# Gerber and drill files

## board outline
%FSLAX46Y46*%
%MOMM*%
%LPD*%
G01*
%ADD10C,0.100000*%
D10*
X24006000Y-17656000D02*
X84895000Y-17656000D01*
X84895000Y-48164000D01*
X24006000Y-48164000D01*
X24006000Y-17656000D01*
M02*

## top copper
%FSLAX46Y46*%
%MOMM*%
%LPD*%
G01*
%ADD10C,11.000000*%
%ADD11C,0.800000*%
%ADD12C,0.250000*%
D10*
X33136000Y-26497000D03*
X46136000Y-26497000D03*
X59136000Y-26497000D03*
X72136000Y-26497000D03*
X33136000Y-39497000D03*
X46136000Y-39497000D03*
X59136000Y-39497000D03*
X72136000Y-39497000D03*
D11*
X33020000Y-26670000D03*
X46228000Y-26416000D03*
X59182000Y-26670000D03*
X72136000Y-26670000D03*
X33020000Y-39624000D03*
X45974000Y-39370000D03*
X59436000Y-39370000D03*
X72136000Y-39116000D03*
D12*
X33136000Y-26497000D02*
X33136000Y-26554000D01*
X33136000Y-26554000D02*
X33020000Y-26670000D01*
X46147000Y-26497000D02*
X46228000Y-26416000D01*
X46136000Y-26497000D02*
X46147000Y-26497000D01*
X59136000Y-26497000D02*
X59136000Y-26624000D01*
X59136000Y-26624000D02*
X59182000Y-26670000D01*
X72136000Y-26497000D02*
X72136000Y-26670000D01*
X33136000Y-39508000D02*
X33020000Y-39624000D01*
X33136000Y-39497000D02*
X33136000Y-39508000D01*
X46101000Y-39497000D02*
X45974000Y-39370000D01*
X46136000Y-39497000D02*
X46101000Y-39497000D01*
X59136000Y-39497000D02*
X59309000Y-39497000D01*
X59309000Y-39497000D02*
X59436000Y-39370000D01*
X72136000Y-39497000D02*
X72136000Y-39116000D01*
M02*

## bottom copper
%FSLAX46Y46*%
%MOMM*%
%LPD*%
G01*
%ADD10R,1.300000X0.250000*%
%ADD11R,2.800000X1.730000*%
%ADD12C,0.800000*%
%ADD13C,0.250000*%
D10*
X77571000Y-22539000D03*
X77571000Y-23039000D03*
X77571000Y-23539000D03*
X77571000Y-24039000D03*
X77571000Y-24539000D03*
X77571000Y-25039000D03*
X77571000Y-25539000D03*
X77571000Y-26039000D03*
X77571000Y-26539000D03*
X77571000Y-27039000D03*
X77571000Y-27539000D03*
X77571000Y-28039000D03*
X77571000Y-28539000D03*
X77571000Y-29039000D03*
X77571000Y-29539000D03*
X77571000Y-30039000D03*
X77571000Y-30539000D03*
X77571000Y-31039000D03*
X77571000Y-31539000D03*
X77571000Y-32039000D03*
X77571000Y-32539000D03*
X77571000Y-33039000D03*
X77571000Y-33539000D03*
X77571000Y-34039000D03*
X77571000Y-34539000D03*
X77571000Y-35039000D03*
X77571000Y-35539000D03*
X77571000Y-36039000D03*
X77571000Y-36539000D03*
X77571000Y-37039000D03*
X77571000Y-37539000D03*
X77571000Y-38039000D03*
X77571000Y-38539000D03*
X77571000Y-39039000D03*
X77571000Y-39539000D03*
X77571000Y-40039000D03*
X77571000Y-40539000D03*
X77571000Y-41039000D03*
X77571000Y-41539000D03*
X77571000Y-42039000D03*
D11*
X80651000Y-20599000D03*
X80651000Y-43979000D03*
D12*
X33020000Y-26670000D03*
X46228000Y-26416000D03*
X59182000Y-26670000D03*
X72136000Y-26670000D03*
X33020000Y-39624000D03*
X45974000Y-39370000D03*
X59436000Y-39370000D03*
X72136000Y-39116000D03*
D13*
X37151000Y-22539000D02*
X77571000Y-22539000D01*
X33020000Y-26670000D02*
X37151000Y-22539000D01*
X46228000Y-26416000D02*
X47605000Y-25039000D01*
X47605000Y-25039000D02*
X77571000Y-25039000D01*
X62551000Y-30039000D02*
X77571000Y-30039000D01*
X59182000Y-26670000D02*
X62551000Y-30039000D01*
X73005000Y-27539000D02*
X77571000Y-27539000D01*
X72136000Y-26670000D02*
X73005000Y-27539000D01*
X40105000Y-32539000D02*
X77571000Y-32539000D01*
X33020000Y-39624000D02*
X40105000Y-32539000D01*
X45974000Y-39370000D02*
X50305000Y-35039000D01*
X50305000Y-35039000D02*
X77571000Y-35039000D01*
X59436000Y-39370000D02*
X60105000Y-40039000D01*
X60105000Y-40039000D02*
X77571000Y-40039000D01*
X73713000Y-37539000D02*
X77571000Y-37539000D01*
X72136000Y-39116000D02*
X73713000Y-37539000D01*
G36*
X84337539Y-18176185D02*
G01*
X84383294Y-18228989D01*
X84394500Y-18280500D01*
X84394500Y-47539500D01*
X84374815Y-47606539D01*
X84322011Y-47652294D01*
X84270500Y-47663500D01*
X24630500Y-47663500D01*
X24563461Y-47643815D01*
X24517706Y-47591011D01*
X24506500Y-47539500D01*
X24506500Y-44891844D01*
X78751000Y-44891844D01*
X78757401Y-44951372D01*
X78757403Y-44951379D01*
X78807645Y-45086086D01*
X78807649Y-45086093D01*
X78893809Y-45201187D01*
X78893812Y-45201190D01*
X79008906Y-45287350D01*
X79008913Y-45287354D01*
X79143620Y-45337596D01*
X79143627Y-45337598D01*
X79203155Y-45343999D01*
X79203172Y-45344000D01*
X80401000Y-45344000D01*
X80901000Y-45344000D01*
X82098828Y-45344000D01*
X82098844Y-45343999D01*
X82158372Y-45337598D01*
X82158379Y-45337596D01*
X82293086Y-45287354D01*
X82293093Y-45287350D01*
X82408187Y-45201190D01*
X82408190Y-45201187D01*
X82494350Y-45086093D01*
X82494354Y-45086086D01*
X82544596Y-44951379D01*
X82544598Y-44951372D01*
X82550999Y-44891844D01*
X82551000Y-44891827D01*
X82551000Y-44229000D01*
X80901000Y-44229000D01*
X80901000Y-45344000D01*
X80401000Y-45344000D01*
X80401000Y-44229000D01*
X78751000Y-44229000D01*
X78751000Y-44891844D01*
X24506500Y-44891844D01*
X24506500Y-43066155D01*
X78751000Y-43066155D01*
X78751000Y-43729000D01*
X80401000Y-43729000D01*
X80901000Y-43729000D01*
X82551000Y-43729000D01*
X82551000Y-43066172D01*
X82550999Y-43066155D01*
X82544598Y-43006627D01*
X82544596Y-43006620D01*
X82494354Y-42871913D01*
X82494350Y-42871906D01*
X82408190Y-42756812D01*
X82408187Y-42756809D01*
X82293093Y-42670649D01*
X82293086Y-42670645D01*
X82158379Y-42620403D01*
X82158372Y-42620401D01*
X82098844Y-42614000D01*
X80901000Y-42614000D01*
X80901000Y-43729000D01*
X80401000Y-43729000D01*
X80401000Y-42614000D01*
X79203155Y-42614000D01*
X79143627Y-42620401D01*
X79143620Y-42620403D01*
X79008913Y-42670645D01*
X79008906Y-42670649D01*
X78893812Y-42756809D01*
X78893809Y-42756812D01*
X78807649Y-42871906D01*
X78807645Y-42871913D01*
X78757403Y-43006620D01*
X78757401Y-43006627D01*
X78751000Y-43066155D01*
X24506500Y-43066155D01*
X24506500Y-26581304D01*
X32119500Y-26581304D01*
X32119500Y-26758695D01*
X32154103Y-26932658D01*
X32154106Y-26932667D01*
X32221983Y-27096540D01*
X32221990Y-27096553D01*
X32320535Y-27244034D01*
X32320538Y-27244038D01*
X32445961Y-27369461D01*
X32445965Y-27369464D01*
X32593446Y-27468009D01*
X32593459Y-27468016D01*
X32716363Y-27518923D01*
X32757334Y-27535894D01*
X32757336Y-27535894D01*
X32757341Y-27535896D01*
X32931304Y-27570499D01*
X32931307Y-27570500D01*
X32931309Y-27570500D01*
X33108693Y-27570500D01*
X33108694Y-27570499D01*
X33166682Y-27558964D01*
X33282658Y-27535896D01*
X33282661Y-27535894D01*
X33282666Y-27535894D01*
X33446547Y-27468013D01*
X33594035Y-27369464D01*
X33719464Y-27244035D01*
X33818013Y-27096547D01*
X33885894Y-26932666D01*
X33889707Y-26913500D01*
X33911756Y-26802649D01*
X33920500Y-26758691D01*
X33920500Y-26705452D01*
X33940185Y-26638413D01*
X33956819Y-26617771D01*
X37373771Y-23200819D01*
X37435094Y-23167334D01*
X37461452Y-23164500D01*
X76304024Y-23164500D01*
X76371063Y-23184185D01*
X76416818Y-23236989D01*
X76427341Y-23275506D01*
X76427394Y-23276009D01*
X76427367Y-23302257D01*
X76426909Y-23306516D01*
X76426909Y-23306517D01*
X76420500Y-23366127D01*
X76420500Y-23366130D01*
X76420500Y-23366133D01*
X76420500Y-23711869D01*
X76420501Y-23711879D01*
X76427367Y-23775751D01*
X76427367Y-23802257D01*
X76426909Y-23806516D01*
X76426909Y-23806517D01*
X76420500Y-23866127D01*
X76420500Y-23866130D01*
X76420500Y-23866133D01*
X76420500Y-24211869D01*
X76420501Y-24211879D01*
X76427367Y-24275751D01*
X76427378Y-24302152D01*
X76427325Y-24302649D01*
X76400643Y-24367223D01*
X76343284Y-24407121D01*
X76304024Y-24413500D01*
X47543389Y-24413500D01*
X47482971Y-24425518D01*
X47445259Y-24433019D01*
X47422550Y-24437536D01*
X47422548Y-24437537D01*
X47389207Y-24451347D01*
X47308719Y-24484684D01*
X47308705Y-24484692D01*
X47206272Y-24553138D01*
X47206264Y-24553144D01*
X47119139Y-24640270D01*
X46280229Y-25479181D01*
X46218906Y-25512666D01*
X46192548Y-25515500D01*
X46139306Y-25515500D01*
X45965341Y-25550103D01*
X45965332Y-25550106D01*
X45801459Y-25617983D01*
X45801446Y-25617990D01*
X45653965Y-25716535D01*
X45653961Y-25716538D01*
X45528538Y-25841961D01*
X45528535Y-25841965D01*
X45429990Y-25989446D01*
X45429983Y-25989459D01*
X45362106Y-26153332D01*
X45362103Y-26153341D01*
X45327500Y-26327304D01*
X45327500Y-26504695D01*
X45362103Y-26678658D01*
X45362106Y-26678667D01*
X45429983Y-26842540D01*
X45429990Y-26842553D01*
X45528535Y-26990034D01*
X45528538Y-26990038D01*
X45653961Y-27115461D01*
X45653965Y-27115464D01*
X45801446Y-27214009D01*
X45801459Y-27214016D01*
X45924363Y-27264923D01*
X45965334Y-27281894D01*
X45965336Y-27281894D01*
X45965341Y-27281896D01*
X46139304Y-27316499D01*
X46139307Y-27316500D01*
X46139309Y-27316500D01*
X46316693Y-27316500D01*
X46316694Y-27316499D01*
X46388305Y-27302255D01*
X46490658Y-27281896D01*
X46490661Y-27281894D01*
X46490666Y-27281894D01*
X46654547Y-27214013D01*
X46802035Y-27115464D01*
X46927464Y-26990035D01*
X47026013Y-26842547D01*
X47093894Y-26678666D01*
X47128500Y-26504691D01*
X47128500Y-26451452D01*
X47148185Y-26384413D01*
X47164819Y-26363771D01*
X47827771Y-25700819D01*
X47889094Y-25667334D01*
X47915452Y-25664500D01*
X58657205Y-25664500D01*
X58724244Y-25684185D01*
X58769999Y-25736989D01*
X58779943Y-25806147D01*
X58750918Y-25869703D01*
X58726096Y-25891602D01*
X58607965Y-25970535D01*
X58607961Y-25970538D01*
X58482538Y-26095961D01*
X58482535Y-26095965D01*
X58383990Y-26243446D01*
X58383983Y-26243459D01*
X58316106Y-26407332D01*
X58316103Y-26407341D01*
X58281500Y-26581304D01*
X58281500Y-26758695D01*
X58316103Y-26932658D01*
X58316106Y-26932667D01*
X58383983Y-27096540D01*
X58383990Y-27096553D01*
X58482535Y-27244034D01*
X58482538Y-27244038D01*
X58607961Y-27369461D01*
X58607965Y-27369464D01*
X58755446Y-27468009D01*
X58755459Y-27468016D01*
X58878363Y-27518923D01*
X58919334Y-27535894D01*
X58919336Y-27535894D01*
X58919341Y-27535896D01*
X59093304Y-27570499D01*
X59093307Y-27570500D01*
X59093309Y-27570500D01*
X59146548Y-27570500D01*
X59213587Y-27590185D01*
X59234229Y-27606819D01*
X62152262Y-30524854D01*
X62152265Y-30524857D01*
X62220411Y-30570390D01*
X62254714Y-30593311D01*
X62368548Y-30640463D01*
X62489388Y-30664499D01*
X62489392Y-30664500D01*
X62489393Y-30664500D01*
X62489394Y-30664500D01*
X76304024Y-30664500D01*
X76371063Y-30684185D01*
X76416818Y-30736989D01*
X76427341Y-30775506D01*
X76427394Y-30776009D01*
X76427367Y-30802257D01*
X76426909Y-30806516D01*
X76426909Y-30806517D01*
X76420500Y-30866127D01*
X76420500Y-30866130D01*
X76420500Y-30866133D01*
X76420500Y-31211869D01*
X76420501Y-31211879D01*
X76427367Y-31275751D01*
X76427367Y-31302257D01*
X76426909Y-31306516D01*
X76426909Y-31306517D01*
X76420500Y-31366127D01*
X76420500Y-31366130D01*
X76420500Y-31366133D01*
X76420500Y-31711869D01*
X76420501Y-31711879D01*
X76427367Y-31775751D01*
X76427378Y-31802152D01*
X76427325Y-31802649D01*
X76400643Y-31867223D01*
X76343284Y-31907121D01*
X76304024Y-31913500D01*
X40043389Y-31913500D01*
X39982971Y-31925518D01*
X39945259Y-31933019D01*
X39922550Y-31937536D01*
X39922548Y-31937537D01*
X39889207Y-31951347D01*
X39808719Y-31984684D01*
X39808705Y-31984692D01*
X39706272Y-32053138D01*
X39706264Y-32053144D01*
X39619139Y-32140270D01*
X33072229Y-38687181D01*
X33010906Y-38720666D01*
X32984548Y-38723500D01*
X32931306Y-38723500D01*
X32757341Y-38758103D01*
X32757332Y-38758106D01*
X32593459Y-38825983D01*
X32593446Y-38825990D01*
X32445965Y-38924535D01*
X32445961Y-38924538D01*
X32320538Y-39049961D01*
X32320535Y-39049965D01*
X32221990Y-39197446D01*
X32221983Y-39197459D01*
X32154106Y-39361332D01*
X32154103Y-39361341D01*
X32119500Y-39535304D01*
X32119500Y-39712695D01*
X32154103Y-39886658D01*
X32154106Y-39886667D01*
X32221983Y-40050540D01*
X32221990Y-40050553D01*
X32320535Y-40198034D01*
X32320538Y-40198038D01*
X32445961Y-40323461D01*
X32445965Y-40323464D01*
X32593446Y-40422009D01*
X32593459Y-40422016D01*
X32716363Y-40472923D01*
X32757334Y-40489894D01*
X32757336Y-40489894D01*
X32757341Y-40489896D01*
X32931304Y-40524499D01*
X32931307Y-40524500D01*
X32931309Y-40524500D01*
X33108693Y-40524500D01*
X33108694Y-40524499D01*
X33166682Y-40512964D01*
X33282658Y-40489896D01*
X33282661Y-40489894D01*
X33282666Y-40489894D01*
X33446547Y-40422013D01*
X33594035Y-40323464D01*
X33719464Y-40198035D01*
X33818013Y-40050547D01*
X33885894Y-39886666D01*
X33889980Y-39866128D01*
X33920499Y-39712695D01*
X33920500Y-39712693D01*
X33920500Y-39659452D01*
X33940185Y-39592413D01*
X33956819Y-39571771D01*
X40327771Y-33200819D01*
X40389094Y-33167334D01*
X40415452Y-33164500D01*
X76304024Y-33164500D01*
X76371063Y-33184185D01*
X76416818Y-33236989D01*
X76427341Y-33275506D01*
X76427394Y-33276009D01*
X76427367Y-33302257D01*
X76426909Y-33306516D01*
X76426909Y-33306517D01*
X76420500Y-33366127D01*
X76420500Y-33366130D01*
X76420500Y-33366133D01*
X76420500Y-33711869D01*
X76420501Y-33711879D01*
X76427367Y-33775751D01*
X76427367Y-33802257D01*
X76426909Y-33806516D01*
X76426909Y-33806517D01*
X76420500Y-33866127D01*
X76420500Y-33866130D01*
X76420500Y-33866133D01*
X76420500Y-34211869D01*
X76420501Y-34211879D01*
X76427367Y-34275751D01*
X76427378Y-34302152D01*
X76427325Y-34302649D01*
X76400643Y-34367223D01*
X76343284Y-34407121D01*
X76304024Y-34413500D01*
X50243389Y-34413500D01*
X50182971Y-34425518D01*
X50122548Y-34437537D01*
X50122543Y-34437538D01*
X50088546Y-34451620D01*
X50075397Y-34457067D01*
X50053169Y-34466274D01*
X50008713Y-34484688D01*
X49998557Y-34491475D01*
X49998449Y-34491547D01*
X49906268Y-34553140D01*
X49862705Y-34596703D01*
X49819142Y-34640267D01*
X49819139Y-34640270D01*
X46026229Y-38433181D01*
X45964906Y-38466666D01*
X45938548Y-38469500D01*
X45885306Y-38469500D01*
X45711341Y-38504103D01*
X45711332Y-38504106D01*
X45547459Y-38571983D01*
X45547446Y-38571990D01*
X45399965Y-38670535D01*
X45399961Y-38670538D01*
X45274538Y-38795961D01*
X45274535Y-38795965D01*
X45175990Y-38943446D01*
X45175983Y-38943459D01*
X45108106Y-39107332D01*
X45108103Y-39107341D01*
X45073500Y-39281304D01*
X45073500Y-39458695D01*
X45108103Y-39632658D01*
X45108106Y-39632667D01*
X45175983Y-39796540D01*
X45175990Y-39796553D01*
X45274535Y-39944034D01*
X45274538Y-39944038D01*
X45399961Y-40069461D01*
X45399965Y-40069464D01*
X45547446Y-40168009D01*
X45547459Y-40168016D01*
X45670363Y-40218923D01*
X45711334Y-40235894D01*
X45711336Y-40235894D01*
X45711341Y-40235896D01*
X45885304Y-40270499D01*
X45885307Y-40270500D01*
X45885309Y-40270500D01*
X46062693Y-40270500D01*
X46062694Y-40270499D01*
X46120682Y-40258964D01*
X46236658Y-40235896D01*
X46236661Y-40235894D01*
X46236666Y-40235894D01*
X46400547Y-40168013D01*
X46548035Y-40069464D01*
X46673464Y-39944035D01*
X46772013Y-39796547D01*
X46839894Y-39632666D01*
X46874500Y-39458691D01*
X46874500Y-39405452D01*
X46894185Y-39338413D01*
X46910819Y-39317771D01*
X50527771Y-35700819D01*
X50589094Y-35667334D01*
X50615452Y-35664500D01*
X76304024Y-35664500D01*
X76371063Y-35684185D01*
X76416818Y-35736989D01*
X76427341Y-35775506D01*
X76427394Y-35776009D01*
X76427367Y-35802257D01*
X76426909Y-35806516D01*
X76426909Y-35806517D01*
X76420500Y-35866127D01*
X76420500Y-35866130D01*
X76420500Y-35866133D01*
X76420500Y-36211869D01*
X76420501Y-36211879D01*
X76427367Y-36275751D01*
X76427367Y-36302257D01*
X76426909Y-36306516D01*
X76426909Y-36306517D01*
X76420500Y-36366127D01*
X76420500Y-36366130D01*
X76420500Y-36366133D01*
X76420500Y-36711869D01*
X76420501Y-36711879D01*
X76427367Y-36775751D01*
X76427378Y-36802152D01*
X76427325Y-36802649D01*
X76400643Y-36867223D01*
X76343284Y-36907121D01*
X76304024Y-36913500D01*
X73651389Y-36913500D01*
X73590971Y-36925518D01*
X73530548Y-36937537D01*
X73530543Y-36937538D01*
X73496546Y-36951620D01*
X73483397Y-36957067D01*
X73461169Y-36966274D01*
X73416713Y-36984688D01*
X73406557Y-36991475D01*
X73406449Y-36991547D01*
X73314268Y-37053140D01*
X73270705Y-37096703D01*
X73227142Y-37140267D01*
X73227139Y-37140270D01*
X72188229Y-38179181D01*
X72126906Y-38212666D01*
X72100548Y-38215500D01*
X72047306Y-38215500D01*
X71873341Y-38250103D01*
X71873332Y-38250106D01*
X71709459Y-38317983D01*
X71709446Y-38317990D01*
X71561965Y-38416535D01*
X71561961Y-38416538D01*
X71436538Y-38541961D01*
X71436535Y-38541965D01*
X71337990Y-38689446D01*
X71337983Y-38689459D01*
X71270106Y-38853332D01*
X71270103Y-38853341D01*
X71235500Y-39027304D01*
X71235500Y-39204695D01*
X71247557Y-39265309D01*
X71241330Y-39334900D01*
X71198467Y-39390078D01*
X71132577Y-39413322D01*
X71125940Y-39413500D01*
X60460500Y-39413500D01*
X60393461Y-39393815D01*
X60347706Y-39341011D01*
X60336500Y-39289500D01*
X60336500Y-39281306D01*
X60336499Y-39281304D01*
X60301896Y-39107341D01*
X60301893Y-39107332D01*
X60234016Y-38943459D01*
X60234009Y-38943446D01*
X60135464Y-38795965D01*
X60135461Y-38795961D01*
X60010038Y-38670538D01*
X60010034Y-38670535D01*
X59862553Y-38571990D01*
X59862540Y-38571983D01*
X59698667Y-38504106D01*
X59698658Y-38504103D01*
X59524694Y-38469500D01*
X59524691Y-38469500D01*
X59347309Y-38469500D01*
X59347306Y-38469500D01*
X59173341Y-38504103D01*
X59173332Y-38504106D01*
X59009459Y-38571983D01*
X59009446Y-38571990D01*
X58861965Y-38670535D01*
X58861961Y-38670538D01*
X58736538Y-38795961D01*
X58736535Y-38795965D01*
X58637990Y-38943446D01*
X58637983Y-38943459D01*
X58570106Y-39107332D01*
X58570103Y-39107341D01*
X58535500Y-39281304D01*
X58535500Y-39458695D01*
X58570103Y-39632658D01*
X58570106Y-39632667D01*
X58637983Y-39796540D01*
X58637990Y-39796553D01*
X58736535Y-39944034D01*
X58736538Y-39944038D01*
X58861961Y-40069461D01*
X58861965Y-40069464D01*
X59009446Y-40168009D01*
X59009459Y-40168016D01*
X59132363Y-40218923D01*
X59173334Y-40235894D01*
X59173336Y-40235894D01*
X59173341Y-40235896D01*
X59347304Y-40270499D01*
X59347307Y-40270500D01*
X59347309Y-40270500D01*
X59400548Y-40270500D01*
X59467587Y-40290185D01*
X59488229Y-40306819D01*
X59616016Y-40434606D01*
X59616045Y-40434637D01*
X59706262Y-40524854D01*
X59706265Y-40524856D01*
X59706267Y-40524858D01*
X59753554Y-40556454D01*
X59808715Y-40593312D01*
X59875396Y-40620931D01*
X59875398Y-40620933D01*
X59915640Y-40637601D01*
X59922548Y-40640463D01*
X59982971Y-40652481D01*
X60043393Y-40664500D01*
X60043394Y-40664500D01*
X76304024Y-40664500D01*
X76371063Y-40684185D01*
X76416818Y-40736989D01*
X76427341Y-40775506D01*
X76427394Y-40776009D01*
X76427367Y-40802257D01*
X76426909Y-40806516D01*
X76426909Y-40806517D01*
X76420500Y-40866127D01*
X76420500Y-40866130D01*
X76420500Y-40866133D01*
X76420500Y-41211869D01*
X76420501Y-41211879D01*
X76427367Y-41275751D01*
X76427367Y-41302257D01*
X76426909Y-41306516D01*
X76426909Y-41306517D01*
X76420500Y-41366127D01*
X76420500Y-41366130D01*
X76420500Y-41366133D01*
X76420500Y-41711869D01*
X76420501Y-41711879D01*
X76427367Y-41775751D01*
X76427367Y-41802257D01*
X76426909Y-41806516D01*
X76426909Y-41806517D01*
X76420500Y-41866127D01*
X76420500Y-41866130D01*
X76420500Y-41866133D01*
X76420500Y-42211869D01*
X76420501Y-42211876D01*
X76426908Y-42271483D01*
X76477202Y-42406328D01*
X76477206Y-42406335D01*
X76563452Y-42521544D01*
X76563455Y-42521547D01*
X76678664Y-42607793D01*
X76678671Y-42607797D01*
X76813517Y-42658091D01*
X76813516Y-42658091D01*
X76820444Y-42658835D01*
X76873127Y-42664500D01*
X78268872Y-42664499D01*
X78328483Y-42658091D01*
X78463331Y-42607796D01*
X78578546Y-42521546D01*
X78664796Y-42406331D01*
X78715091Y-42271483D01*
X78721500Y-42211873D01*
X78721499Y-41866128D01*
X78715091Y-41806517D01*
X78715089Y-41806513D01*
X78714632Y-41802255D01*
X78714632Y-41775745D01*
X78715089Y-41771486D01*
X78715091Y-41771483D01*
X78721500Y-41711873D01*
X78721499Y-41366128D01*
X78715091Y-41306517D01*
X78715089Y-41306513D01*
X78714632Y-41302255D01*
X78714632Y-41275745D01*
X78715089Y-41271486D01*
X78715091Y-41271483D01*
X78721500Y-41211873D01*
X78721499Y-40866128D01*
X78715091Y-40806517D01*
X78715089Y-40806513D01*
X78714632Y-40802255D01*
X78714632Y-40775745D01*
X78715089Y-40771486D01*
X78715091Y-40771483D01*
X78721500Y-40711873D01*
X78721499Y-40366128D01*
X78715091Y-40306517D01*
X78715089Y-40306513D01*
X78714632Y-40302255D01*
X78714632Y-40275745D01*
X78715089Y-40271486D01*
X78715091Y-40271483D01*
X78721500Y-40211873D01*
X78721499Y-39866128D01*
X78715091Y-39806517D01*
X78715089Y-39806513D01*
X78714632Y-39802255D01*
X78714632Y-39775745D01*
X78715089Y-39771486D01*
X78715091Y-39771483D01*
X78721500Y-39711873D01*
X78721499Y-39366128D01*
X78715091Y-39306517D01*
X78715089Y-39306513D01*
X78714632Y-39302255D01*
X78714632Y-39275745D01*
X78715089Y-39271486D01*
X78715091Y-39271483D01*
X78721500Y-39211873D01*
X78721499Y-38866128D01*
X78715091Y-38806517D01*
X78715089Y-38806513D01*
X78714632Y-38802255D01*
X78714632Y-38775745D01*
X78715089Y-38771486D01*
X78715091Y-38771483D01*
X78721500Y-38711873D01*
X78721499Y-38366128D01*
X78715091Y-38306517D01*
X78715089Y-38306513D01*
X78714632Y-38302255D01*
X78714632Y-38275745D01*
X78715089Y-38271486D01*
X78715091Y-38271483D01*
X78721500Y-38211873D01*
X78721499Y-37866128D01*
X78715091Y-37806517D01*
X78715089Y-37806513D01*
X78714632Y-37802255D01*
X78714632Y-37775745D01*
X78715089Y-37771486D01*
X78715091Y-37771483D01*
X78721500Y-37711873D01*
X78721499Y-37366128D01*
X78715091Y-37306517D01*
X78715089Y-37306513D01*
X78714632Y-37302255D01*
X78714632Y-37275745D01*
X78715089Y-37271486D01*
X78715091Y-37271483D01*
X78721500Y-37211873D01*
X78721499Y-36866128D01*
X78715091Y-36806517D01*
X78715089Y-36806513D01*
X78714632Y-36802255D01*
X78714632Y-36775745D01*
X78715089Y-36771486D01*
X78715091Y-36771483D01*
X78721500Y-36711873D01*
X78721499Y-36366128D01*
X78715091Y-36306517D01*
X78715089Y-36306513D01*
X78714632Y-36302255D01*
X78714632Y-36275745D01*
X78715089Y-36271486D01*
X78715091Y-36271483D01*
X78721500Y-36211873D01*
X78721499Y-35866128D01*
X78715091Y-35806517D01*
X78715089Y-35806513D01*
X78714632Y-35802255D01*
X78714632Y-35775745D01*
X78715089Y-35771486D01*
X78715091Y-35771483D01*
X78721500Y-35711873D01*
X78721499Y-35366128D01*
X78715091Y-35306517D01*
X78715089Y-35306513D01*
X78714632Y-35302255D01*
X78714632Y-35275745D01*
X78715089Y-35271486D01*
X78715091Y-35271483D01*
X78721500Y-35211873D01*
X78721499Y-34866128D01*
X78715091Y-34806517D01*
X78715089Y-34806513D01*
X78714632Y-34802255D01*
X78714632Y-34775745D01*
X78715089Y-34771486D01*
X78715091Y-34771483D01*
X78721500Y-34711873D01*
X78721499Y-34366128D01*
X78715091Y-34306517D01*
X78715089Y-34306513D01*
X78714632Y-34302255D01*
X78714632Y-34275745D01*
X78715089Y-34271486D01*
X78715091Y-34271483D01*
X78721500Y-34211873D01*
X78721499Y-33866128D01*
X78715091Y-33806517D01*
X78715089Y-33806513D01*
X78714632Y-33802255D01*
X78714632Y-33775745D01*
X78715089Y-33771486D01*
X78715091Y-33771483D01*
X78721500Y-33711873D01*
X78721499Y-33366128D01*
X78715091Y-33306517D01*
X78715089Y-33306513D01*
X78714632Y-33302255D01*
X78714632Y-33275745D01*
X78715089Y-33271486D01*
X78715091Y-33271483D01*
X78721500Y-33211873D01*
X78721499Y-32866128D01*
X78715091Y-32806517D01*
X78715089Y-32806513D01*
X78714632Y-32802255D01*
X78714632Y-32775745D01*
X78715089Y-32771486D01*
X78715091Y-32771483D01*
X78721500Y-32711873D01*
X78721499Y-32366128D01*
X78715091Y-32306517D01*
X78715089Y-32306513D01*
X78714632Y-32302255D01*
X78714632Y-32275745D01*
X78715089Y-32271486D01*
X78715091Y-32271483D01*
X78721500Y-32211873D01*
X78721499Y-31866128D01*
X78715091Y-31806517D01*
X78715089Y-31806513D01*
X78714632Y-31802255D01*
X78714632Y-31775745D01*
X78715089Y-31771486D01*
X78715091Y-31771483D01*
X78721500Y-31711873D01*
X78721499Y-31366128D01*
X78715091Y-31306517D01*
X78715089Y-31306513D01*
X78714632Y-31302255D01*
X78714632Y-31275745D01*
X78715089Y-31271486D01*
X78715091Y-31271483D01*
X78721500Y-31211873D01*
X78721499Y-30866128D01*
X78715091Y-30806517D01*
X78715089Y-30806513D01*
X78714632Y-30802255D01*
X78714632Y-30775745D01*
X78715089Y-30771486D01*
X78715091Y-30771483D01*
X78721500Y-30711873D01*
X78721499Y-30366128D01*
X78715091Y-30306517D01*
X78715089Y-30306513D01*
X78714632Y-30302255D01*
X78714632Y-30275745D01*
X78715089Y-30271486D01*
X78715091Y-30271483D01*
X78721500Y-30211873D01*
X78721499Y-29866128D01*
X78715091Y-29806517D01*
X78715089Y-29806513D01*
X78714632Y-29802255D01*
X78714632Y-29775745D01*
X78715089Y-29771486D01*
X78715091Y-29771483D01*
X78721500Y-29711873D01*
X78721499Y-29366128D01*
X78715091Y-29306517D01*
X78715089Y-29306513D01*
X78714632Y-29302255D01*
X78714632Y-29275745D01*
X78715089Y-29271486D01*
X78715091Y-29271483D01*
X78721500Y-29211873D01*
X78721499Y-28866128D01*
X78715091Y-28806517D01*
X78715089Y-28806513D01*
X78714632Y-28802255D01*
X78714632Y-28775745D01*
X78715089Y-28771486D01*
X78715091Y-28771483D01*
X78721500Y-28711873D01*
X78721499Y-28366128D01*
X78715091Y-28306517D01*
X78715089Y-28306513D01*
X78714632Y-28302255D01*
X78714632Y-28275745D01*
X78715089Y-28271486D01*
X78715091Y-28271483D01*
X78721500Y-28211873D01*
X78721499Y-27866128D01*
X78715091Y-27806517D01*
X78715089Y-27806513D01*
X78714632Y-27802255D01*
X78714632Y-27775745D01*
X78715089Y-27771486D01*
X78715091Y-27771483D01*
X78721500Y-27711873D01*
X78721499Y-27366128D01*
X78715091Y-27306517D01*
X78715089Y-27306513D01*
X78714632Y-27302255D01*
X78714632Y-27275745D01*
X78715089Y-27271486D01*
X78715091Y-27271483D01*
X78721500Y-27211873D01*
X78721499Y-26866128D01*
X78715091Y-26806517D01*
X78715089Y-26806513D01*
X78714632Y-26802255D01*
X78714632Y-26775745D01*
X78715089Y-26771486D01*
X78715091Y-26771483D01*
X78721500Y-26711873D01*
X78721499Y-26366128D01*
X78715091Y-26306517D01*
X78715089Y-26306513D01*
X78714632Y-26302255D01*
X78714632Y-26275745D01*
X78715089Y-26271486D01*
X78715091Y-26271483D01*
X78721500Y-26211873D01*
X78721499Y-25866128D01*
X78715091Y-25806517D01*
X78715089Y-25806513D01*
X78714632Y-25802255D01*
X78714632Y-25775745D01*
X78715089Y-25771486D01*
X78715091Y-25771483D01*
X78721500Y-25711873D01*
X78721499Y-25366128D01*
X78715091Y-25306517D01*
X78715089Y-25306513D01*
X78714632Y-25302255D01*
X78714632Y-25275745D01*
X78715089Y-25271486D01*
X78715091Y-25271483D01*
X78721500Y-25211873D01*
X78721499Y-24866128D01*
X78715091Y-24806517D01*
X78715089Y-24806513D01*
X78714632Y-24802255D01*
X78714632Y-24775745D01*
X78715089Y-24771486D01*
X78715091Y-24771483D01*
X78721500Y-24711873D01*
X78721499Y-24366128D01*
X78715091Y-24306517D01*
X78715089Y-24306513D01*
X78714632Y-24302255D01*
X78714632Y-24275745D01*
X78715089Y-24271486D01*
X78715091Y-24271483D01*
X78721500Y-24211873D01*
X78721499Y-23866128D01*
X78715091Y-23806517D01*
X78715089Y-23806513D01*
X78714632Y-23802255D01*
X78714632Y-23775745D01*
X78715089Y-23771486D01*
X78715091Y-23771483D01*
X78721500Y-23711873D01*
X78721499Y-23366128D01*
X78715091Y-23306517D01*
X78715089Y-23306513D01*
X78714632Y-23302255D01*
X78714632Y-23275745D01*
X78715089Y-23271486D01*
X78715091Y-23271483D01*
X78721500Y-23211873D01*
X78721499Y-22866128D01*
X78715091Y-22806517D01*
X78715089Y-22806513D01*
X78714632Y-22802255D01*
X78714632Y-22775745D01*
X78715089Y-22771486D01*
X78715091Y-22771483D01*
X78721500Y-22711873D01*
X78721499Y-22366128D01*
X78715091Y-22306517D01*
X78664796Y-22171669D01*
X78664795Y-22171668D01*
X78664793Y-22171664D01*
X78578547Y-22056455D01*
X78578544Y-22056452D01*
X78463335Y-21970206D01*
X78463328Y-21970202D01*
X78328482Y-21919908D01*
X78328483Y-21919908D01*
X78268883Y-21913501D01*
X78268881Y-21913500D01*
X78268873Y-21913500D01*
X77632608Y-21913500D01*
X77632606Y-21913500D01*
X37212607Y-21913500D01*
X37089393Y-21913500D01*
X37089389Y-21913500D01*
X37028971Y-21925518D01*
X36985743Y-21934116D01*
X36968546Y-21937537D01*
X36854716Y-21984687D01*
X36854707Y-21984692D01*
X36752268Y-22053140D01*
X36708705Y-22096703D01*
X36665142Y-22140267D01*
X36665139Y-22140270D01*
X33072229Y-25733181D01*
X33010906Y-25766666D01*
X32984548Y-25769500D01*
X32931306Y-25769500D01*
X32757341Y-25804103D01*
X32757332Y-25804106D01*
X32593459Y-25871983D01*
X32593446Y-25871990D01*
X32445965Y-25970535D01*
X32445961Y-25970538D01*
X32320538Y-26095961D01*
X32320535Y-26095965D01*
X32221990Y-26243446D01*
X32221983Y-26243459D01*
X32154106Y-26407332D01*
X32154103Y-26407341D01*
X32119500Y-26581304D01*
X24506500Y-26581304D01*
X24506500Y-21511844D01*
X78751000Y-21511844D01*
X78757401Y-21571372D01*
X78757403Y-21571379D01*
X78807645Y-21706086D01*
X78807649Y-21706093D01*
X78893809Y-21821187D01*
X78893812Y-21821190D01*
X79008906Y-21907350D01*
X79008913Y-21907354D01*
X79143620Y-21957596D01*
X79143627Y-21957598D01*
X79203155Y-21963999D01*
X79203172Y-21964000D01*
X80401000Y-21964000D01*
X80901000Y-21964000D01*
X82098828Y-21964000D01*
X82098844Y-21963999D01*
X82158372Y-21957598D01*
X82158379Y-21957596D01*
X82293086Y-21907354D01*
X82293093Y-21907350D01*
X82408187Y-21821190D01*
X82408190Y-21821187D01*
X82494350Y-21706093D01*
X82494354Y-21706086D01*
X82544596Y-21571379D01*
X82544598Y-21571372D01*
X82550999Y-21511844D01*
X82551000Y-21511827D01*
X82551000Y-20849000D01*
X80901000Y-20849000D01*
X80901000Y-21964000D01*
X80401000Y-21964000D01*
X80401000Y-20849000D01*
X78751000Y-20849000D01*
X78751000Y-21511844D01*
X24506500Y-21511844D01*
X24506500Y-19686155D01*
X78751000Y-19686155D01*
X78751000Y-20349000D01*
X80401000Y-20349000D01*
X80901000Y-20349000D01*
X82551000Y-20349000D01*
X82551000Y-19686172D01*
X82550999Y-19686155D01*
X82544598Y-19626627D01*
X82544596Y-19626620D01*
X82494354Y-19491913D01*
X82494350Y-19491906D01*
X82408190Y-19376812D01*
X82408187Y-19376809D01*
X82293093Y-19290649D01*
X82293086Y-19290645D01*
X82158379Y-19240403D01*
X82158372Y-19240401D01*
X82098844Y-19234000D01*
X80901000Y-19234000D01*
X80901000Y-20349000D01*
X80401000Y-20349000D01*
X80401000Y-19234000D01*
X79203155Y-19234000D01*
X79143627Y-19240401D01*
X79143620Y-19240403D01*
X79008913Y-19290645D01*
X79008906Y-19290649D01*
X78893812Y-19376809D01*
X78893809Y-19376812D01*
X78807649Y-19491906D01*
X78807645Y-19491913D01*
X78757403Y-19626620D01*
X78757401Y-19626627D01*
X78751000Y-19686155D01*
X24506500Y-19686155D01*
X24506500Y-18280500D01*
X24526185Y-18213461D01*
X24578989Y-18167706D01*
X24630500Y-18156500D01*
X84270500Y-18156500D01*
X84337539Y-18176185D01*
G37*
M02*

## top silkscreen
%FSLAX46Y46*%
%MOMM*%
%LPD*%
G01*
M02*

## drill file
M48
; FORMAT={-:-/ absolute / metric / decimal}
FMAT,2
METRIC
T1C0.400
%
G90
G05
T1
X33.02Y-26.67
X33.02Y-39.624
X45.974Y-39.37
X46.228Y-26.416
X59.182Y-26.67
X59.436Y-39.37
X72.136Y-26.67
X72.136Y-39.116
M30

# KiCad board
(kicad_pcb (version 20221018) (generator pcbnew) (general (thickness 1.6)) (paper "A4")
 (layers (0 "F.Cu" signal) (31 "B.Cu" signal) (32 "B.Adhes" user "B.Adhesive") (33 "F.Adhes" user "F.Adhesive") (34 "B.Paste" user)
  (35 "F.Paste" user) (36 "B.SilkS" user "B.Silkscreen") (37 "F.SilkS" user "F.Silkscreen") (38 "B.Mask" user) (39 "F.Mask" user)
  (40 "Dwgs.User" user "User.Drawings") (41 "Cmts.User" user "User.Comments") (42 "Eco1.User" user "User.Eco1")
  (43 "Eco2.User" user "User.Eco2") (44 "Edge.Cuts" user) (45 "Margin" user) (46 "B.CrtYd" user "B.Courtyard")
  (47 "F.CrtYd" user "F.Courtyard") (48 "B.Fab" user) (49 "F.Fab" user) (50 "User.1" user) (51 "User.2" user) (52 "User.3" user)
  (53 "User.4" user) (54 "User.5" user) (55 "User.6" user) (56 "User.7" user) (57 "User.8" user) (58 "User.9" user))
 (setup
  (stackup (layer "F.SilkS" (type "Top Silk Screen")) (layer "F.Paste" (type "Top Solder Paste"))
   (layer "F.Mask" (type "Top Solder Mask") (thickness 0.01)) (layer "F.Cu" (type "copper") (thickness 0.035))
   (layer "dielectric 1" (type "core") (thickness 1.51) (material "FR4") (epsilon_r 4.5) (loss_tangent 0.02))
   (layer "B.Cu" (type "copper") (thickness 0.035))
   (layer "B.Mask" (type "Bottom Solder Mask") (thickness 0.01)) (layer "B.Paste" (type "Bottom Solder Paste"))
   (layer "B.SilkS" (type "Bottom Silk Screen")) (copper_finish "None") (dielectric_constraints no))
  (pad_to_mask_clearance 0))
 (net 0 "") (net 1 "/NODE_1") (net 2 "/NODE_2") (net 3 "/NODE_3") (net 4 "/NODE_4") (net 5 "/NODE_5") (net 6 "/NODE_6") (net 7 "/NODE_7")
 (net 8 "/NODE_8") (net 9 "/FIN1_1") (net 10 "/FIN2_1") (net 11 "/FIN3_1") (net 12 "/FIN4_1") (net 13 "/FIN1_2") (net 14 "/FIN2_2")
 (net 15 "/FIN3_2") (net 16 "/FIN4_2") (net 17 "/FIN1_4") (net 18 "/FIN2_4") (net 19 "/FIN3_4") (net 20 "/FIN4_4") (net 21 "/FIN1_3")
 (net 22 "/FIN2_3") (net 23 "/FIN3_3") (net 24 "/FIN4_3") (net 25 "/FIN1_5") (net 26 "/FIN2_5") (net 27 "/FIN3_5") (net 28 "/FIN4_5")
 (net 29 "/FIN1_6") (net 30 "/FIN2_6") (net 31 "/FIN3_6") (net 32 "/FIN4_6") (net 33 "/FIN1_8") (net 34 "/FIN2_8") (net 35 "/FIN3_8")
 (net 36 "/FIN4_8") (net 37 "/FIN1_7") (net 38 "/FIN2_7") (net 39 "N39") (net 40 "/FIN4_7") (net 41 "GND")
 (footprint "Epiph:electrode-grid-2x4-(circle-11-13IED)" (layer "F.Cu") (at 52.451 33.782)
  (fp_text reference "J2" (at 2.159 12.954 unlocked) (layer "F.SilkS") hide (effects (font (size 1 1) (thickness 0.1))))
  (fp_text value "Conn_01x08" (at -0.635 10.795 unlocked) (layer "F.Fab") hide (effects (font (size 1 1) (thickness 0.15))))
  (pad "1" smd circle (at -19.315 -7.285) (size 11 11) (layers "F.Cu" "F.Paste" "F.Mask") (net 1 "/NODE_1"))
  (pad "2" smd circle (at -6.315 -7.285) (size 11 11) (layers "F.Cu" "F.Paste" "F.Mask") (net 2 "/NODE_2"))
  (pad "3" smd circle (at 6.685 -7.285) (size 11 11) (layers "F.Cu" "F.Paste" "F.Mask") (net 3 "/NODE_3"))
  (pad "4" smd circle (at 19.685 -7.285) (size 11 11) (layers "F.Cu" "F.Paste" "F.Mask") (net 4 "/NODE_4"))
  (pad "5" smd circle (at -19.315 5.715) (size 11 11) (layers "F.Cu" "F.Paste" "F.Mask") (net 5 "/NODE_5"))
  (pad "6" smd circle (at -6.315 5.715) (size 11 11) (layers "F.Cu" "F.Paste" "F.Mask") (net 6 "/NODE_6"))
  (pad "7" smd circle (at 6.685 5.715) (size 11 11) (layers "F.Cu" "F.Paste" "F.Mask") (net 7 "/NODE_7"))
  (pad "8" smd circle (at 19.685 5.715) (size 11 11) (layers "F.Cu" "F.Paste" "F.Mask") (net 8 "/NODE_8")))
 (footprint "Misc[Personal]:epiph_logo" (layer "B.Cu") (at 43.18 23.876 180)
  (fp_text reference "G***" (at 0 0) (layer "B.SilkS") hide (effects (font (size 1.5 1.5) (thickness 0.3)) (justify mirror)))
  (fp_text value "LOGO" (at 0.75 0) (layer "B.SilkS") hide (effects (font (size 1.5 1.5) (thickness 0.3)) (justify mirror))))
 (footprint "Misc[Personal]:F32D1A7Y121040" (layer "B.Cu") (at 80.041 32.289 -90)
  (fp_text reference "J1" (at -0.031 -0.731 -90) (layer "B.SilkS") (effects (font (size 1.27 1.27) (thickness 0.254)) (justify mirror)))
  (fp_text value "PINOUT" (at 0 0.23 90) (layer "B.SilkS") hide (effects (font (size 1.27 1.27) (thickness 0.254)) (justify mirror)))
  (pad "1" smd rect (at -9.75 2.47 270) (size 0.25 1.3) (layers "B.Cu" "B.Paste" "B.Mask") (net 1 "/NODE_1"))
  (pad "2" smd rect (at -9.25 2.47 270) (size 0.25 1.3) (layers "B.Cu" "B.Paste" "B.Mask") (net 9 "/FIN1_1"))
  (pad "3" smd rect (at -8.75 2.47 270) (size 0.25 1.3) (layers "B.Cu" "B.Paste" "B.Mask") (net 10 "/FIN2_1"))
  (pad "4" smd rect (at -8.25 2.47 270) (size 0.25 1.3) (layers "B.Cu" "B.Paste" "B.Mask") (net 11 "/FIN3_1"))
  (pad "5" smd rect (at -7.75 2.47 270) (size 0.25 1.3) (layers "B.Cu" "B.Paste" "B.Mask") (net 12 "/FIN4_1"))
  (pad "6" smd rect (at -7.25 2.47 270) (size 0.25 1.3) (layers "B.Cu" "B.Paste" "B.Mask") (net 2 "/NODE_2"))
  (pad "7" smd rect (at -6.75 2.47 270) (size 0.25 1.3) (layers "B.Cu" "B.Paste" "B.Mask") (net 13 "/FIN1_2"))
  (pad "8" smd rect (at -6.25 2.47 270) (size 0.25 1.3) (layers "B.Cu" "B.Paste" "B.Mask") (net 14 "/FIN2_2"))
  (pad "9" smd rect (at -5.75 2.47 270) (size 0.25 1.3) (layers "B.Cu" "B.Paste" "B.Mask") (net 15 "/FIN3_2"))
  (pad "10" smd rect (at -5.25 2.47 270) (size 0.25 1.3) (layers "B.Cu" "B.Paste" "B.Mask") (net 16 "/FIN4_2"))
  (pad "11" smd rect (at -4.75 2.47 270) (size 0.25 1.3) (layers "B.Cu" "B.Paste" "B.Mask") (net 4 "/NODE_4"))
  (pad "12" smd rect (at -4.25 2.47 270) (size 0.25 1.3) (layers "B.Cu" "B.Paste" "B.Mask") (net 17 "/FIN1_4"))
  (pad "13" smd rect (at -3.75 2.47 270) (size 0.25 1.3) (layers "B.Cu" "B.Paste" "B.Mask") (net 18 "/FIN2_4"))
  (pad "14" smd rect (at -3.25 2.47 270) (size 0.25 1.3) (layers "B.Cu" "B.Paste" "B.Mask") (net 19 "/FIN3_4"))
  (pad "15" smd rect (at -2.75 2.47 270) (size 0.25 1.3) (layers "B.Cu" "B.Paste" "B.Mask") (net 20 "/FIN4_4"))
  (pad "16" smd rect (at -2.25 2.47 270) (size 0.25 1.3) (layers "B.Cu" "B.Paste" "B.Mask") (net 3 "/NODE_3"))
  (pad "17" smd rect (at -1.75 2.47 270) (size 0.25 1.3) (layers "B.Cu" "B.Paste" "B.Mask") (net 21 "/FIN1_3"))
  (pad "18" smd rect (at -1.25 2.47 270) (size 0.25 1.3) (layers "B.Cu" "B.Paste" "B.Mask") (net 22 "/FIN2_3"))
  (pad "19" smd rect (at -0.75 2.47 270) (size 0.25 1.3) (layers "B.Cu" "B.Paste" "B.Mask") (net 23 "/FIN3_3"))
  (pad "20" smd rect (at -0.25 2.47 270) (size 0.25 1.3) (layers "B.Cu" "B.Paste" "B.Mask") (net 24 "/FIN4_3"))
  (pad "21" smd rect (at 0.25 2.47 270) (size 0.25 1.3) (layers "B.Cu" "B.Paste" "B.Mask") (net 5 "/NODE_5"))
  (pad "22" smd rect (at 0.75 2.47 270) (size 0.25 1.3) (layers "B.Cu" "B.Paste" "B.Mask") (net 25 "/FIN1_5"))
  (pad "23" smd rect (at 1.25 2.47 270) (size 0.25 1.3) (layers "B.Cu" "B.Paste" "B.Mask") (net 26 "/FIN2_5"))
  (pad "24" smd rect (at 1.75 2.47 270) (size 0.25 1.3) (layers "B.Cu" "B.Paste" "B.Mask") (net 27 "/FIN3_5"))
  (pad "25" smd rect (at 2.25 2.47 270) (size 0.25 1.3) (layers "B.Cu" "B.Paste" "B.Mask") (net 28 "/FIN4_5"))
  (pad "26" smd rect (at 2.75 2.47 270) (size 0.25 1.3) (layers "B.Cu" "B.Paste" "B.Mask") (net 6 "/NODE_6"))
  (pad "27" smd rect (at 3.25 2.47 270) (size 0.25 1.3) (layers "B.Cu" "B.Paste" "B.Mask") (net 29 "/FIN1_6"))
  (pad "28" smd rect (at 3.75 2.47 270) (size 0.25 1.3) (layers "B.Cu" "B.Paste" "B.Mask") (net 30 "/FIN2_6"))
  (pad "29" smd rect (at 4.25 2.47 270) (size 0.25 1.3) (layers "B.Cu" "B.Paste" "B.Mask") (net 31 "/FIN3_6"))
  (pad "30" smd rect (at 4.75 2.47 270) (size 0.25 1.3) (layers "B.Cu" "B.Paste" "B.Mask") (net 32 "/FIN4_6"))
  (pad "31" smd rect (at 5.25 2.47 270) (size 0.25 1.3) (layers "B.Cu" "B.Paste" "B.Mask") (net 8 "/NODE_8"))
  (pad "32" smd rect (at 5.75 2.47 270) (size 0.25 1.3) (layers "B.Cu" "B.Paste" "B.Mask") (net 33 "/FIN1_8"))
  (pad "33" smd rect (at 6.25 2.47 270) (size 0.25 1.3) (layers "B.Cu" "B.Paste" "B.Mask") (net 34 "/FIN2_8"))
  (pad "34" smd rect (at 6.75 2.47 270) (size 0.25 1.3) (layers "B.Cu" "B.Paste" "B.Mask") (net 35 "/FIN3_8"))
  (pad "35" smd rect (at 7.25 2.47 270) (size 0.25 1.3) (layers "B.Cu" "B.Paste" "B.Mask") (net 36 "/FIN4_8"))
  (pad "36" smd rect (at 7.75 2.47 270) (size 0.25 1.3) (layers "B.Cu" "B.Paste" "B.Mask") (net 7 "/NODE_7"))
  (pad "37" smd rect (at 8.25 2.47 270) (size 0.25 1.3) (layers "B.Cu" "B.Paste" "B.Mask") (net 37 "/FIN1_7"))
  (pad "38" smd rect (at 8.75 2.47 270) (size 0.25 1.3) (layers "B.Cu" "B.Paste" "B.Mask") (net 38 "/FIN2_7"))
  (pad "39" smd rect (at 9.25 2.47 270) (size 0.25 1.3) (layers "B.Cu" "B.Paste" "B.Mask") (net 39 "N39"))
  (pad "40" smd rect (at 9.75 2.47 270) (size 0.25 1.3) (layers "B.Cu" "B.Paste" "B.Mask") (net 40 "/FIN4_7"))
  (pad "MP1" smd rect (at -11.69 -0.61 270) (size 1.73 2.8) (layers "B.Cu" "B.Paste" "B.Mask") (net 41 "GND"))
  (pad "MP2" smd rect (at 11.69 -0.61 270) (size 1.73 2.8) (layers "B.Cu" "B.Paste" "B.Mask") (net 41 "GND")))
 (gr_rect (start 24.006 17.656) (end 84.895 48.164) (stroke (width 0.1) (type default)) (fill none) (layer "Edge.Cuts"))
 (segment (start 33.136 26.497) (end 33.136 26.554) (width 0.25) (layer "F.Cu") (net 1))
 (segment (start 33.136 26.554) (end 33.02 26.67) (width 0.25) (layer "F.Cu") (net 1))
 (via (at 33.02 26.67) (size 0.8) (drill 0.4) (layers "F.Cu" "B.Cu") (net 1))
 (segment (start 37.151 22.539) (end 77.571 22.539) (width 0.25) (layer "B.Cu") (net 1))
 (segment (start 33.02 26.67) (end 37.151 22.539) (width 0.25) (layer "B.Cu") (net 1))
 (segment (start 46.147 26.497) (end 46.228 26.416) (width 0.25) (layer "F.Cu") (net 2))
 (segment (start 46.136 26.497) (end 46.147 26.497) (width 0.25) (layer "F.Cu") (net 2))
 (via (at 46.228 26.416) (size 0.8) (drill 0.4) (layers "F.Cu" "B.Cu") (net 2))
 (segment (start 46.228 26.416) (end 47.605 25.039) (width 0.25) (layer "B.Cu") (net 2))
 (segment (start 47.605 25.039) (end 77.571 25.039) (width 0.25) (layer "B.Cu") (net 2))
 (segment (start 59.136 26.497) (end 59.136 26.624) (width 0.25) (layer "F.Cu") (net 3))
 (segment (start 59.136 26.624) (end 59.182 26.67) (width 0.25) (layer "F.Cu") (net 3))
 (via (at 59.182 26.67) (size 0.8) (drill 0.4) (layers "F.Cu" "B.Cu") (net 3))
 (segment (start 62.551 30.039) (end 77.571 30.039) (width 0.25) (layer "B.Cu") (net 3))
 (segment (start 59.182 26.67) (end 62.551 30.039) (width 0.25) (layer "B.Cu") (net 3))
 (segment (start 72.136 26.497) (end 72.136 26.67) (width 0.25) (layer "F.Cu") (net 4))
 (via (at 72.136 26.67) (size 0.8) (drill 0.4) (layers "F.Cu" "B.Cu") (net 4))
 (segment (start 73.005 27.539) (end 77.571 27.539) (width 0.25) (layer "B.Cu") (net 4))
 (segment (start 72.136 26.67) (end 73.005 27.539) (width 0.25) (layer "B.Cu") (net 4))
 (segment (start 33.136 39.508) (end 33.02 39.624) (width 0.25) (layer "F.Cu") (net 5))
 (segment (start 33.136 39.497) (end 33.136 39.508) (width 0.25) (layer "F.Cu") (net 5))
 (via (at 33.02 39.624) (size 0.8) (drill 0.4) (layers "F.Cu" "B.Cu") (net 5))
 (segment (start 40.105 32.539) (end 77.571 32.539) (width 0.25) (layer "B.Cu") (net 5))
 (segment (start 33.02 39.624) (end 40.105 32.539) (width 0.25) (layer "B.Cu") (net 5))
 (segment (start 46.101 39.497) (end 45.974 39.37) (width 0.25) (layer "F.Cu") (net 6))
 (segment (start 46.136 39.497) (end 46.101 39.497) (width 0.25) (layer "F.Cu") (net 6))
 (via (at 45.974 39.37) (size 0.8) (drill 0.4) (layers "F.Cu" "B.Cu") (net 6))
 (segment (start 45.974 39.37) (end 50.305 35.039) (width 0.25) (layer "B.Cu") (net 6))
 (segment (start 50.305 35.039) (end 77.571 35.039) (width 0.25) (layer "B.Cu") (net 6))
 (segment (start 59.136 39.497) (end 59.309 39.497) (width 0.25) (layer "F.Cu") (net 7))
 (segment (start 59.309 39.497) (end 59.436 39.37) (width 0.25) (layer "F.Cu") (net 7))
 (via (at 59.436 39.37) (size 0.8) (drill 0.4) (layers "F.Cu" "B.Cu") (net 7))
 (segment (start 59.436 39.37) (end 60.105 40.039) (width 0.25) (layer "B.Cu") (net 7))
 (segment (start 60.105 40.039) (end 77.571 40.039) (width 0.25) (layer "B.Cu") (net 7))
 (segment (start 72.136 39.497) (end 72.136 39.116) (width 0.25) (layer "F.Cu") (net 8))
 (via (at 72.136 39.116) (size 0.8) (drill 0.4) (layers "F.Cu" "B.Cu") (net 8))
 (segment (start 73.713 37.539) (end 77.571 37.539) (width 0.25) (layer "B.Cu") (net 8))
 (segment (start 72.136 39.116) (end 73.713 37.539) (width 0.25) (layer "B.Cu") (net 8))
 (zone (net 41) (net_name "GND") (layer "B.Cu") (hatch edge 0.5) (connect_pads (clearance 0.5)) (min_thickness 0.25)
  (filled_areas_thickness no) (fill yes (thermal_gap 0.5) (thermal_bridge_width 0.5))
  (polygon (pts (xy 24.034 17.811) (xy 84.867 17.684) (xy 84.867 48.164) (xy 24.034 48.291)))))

